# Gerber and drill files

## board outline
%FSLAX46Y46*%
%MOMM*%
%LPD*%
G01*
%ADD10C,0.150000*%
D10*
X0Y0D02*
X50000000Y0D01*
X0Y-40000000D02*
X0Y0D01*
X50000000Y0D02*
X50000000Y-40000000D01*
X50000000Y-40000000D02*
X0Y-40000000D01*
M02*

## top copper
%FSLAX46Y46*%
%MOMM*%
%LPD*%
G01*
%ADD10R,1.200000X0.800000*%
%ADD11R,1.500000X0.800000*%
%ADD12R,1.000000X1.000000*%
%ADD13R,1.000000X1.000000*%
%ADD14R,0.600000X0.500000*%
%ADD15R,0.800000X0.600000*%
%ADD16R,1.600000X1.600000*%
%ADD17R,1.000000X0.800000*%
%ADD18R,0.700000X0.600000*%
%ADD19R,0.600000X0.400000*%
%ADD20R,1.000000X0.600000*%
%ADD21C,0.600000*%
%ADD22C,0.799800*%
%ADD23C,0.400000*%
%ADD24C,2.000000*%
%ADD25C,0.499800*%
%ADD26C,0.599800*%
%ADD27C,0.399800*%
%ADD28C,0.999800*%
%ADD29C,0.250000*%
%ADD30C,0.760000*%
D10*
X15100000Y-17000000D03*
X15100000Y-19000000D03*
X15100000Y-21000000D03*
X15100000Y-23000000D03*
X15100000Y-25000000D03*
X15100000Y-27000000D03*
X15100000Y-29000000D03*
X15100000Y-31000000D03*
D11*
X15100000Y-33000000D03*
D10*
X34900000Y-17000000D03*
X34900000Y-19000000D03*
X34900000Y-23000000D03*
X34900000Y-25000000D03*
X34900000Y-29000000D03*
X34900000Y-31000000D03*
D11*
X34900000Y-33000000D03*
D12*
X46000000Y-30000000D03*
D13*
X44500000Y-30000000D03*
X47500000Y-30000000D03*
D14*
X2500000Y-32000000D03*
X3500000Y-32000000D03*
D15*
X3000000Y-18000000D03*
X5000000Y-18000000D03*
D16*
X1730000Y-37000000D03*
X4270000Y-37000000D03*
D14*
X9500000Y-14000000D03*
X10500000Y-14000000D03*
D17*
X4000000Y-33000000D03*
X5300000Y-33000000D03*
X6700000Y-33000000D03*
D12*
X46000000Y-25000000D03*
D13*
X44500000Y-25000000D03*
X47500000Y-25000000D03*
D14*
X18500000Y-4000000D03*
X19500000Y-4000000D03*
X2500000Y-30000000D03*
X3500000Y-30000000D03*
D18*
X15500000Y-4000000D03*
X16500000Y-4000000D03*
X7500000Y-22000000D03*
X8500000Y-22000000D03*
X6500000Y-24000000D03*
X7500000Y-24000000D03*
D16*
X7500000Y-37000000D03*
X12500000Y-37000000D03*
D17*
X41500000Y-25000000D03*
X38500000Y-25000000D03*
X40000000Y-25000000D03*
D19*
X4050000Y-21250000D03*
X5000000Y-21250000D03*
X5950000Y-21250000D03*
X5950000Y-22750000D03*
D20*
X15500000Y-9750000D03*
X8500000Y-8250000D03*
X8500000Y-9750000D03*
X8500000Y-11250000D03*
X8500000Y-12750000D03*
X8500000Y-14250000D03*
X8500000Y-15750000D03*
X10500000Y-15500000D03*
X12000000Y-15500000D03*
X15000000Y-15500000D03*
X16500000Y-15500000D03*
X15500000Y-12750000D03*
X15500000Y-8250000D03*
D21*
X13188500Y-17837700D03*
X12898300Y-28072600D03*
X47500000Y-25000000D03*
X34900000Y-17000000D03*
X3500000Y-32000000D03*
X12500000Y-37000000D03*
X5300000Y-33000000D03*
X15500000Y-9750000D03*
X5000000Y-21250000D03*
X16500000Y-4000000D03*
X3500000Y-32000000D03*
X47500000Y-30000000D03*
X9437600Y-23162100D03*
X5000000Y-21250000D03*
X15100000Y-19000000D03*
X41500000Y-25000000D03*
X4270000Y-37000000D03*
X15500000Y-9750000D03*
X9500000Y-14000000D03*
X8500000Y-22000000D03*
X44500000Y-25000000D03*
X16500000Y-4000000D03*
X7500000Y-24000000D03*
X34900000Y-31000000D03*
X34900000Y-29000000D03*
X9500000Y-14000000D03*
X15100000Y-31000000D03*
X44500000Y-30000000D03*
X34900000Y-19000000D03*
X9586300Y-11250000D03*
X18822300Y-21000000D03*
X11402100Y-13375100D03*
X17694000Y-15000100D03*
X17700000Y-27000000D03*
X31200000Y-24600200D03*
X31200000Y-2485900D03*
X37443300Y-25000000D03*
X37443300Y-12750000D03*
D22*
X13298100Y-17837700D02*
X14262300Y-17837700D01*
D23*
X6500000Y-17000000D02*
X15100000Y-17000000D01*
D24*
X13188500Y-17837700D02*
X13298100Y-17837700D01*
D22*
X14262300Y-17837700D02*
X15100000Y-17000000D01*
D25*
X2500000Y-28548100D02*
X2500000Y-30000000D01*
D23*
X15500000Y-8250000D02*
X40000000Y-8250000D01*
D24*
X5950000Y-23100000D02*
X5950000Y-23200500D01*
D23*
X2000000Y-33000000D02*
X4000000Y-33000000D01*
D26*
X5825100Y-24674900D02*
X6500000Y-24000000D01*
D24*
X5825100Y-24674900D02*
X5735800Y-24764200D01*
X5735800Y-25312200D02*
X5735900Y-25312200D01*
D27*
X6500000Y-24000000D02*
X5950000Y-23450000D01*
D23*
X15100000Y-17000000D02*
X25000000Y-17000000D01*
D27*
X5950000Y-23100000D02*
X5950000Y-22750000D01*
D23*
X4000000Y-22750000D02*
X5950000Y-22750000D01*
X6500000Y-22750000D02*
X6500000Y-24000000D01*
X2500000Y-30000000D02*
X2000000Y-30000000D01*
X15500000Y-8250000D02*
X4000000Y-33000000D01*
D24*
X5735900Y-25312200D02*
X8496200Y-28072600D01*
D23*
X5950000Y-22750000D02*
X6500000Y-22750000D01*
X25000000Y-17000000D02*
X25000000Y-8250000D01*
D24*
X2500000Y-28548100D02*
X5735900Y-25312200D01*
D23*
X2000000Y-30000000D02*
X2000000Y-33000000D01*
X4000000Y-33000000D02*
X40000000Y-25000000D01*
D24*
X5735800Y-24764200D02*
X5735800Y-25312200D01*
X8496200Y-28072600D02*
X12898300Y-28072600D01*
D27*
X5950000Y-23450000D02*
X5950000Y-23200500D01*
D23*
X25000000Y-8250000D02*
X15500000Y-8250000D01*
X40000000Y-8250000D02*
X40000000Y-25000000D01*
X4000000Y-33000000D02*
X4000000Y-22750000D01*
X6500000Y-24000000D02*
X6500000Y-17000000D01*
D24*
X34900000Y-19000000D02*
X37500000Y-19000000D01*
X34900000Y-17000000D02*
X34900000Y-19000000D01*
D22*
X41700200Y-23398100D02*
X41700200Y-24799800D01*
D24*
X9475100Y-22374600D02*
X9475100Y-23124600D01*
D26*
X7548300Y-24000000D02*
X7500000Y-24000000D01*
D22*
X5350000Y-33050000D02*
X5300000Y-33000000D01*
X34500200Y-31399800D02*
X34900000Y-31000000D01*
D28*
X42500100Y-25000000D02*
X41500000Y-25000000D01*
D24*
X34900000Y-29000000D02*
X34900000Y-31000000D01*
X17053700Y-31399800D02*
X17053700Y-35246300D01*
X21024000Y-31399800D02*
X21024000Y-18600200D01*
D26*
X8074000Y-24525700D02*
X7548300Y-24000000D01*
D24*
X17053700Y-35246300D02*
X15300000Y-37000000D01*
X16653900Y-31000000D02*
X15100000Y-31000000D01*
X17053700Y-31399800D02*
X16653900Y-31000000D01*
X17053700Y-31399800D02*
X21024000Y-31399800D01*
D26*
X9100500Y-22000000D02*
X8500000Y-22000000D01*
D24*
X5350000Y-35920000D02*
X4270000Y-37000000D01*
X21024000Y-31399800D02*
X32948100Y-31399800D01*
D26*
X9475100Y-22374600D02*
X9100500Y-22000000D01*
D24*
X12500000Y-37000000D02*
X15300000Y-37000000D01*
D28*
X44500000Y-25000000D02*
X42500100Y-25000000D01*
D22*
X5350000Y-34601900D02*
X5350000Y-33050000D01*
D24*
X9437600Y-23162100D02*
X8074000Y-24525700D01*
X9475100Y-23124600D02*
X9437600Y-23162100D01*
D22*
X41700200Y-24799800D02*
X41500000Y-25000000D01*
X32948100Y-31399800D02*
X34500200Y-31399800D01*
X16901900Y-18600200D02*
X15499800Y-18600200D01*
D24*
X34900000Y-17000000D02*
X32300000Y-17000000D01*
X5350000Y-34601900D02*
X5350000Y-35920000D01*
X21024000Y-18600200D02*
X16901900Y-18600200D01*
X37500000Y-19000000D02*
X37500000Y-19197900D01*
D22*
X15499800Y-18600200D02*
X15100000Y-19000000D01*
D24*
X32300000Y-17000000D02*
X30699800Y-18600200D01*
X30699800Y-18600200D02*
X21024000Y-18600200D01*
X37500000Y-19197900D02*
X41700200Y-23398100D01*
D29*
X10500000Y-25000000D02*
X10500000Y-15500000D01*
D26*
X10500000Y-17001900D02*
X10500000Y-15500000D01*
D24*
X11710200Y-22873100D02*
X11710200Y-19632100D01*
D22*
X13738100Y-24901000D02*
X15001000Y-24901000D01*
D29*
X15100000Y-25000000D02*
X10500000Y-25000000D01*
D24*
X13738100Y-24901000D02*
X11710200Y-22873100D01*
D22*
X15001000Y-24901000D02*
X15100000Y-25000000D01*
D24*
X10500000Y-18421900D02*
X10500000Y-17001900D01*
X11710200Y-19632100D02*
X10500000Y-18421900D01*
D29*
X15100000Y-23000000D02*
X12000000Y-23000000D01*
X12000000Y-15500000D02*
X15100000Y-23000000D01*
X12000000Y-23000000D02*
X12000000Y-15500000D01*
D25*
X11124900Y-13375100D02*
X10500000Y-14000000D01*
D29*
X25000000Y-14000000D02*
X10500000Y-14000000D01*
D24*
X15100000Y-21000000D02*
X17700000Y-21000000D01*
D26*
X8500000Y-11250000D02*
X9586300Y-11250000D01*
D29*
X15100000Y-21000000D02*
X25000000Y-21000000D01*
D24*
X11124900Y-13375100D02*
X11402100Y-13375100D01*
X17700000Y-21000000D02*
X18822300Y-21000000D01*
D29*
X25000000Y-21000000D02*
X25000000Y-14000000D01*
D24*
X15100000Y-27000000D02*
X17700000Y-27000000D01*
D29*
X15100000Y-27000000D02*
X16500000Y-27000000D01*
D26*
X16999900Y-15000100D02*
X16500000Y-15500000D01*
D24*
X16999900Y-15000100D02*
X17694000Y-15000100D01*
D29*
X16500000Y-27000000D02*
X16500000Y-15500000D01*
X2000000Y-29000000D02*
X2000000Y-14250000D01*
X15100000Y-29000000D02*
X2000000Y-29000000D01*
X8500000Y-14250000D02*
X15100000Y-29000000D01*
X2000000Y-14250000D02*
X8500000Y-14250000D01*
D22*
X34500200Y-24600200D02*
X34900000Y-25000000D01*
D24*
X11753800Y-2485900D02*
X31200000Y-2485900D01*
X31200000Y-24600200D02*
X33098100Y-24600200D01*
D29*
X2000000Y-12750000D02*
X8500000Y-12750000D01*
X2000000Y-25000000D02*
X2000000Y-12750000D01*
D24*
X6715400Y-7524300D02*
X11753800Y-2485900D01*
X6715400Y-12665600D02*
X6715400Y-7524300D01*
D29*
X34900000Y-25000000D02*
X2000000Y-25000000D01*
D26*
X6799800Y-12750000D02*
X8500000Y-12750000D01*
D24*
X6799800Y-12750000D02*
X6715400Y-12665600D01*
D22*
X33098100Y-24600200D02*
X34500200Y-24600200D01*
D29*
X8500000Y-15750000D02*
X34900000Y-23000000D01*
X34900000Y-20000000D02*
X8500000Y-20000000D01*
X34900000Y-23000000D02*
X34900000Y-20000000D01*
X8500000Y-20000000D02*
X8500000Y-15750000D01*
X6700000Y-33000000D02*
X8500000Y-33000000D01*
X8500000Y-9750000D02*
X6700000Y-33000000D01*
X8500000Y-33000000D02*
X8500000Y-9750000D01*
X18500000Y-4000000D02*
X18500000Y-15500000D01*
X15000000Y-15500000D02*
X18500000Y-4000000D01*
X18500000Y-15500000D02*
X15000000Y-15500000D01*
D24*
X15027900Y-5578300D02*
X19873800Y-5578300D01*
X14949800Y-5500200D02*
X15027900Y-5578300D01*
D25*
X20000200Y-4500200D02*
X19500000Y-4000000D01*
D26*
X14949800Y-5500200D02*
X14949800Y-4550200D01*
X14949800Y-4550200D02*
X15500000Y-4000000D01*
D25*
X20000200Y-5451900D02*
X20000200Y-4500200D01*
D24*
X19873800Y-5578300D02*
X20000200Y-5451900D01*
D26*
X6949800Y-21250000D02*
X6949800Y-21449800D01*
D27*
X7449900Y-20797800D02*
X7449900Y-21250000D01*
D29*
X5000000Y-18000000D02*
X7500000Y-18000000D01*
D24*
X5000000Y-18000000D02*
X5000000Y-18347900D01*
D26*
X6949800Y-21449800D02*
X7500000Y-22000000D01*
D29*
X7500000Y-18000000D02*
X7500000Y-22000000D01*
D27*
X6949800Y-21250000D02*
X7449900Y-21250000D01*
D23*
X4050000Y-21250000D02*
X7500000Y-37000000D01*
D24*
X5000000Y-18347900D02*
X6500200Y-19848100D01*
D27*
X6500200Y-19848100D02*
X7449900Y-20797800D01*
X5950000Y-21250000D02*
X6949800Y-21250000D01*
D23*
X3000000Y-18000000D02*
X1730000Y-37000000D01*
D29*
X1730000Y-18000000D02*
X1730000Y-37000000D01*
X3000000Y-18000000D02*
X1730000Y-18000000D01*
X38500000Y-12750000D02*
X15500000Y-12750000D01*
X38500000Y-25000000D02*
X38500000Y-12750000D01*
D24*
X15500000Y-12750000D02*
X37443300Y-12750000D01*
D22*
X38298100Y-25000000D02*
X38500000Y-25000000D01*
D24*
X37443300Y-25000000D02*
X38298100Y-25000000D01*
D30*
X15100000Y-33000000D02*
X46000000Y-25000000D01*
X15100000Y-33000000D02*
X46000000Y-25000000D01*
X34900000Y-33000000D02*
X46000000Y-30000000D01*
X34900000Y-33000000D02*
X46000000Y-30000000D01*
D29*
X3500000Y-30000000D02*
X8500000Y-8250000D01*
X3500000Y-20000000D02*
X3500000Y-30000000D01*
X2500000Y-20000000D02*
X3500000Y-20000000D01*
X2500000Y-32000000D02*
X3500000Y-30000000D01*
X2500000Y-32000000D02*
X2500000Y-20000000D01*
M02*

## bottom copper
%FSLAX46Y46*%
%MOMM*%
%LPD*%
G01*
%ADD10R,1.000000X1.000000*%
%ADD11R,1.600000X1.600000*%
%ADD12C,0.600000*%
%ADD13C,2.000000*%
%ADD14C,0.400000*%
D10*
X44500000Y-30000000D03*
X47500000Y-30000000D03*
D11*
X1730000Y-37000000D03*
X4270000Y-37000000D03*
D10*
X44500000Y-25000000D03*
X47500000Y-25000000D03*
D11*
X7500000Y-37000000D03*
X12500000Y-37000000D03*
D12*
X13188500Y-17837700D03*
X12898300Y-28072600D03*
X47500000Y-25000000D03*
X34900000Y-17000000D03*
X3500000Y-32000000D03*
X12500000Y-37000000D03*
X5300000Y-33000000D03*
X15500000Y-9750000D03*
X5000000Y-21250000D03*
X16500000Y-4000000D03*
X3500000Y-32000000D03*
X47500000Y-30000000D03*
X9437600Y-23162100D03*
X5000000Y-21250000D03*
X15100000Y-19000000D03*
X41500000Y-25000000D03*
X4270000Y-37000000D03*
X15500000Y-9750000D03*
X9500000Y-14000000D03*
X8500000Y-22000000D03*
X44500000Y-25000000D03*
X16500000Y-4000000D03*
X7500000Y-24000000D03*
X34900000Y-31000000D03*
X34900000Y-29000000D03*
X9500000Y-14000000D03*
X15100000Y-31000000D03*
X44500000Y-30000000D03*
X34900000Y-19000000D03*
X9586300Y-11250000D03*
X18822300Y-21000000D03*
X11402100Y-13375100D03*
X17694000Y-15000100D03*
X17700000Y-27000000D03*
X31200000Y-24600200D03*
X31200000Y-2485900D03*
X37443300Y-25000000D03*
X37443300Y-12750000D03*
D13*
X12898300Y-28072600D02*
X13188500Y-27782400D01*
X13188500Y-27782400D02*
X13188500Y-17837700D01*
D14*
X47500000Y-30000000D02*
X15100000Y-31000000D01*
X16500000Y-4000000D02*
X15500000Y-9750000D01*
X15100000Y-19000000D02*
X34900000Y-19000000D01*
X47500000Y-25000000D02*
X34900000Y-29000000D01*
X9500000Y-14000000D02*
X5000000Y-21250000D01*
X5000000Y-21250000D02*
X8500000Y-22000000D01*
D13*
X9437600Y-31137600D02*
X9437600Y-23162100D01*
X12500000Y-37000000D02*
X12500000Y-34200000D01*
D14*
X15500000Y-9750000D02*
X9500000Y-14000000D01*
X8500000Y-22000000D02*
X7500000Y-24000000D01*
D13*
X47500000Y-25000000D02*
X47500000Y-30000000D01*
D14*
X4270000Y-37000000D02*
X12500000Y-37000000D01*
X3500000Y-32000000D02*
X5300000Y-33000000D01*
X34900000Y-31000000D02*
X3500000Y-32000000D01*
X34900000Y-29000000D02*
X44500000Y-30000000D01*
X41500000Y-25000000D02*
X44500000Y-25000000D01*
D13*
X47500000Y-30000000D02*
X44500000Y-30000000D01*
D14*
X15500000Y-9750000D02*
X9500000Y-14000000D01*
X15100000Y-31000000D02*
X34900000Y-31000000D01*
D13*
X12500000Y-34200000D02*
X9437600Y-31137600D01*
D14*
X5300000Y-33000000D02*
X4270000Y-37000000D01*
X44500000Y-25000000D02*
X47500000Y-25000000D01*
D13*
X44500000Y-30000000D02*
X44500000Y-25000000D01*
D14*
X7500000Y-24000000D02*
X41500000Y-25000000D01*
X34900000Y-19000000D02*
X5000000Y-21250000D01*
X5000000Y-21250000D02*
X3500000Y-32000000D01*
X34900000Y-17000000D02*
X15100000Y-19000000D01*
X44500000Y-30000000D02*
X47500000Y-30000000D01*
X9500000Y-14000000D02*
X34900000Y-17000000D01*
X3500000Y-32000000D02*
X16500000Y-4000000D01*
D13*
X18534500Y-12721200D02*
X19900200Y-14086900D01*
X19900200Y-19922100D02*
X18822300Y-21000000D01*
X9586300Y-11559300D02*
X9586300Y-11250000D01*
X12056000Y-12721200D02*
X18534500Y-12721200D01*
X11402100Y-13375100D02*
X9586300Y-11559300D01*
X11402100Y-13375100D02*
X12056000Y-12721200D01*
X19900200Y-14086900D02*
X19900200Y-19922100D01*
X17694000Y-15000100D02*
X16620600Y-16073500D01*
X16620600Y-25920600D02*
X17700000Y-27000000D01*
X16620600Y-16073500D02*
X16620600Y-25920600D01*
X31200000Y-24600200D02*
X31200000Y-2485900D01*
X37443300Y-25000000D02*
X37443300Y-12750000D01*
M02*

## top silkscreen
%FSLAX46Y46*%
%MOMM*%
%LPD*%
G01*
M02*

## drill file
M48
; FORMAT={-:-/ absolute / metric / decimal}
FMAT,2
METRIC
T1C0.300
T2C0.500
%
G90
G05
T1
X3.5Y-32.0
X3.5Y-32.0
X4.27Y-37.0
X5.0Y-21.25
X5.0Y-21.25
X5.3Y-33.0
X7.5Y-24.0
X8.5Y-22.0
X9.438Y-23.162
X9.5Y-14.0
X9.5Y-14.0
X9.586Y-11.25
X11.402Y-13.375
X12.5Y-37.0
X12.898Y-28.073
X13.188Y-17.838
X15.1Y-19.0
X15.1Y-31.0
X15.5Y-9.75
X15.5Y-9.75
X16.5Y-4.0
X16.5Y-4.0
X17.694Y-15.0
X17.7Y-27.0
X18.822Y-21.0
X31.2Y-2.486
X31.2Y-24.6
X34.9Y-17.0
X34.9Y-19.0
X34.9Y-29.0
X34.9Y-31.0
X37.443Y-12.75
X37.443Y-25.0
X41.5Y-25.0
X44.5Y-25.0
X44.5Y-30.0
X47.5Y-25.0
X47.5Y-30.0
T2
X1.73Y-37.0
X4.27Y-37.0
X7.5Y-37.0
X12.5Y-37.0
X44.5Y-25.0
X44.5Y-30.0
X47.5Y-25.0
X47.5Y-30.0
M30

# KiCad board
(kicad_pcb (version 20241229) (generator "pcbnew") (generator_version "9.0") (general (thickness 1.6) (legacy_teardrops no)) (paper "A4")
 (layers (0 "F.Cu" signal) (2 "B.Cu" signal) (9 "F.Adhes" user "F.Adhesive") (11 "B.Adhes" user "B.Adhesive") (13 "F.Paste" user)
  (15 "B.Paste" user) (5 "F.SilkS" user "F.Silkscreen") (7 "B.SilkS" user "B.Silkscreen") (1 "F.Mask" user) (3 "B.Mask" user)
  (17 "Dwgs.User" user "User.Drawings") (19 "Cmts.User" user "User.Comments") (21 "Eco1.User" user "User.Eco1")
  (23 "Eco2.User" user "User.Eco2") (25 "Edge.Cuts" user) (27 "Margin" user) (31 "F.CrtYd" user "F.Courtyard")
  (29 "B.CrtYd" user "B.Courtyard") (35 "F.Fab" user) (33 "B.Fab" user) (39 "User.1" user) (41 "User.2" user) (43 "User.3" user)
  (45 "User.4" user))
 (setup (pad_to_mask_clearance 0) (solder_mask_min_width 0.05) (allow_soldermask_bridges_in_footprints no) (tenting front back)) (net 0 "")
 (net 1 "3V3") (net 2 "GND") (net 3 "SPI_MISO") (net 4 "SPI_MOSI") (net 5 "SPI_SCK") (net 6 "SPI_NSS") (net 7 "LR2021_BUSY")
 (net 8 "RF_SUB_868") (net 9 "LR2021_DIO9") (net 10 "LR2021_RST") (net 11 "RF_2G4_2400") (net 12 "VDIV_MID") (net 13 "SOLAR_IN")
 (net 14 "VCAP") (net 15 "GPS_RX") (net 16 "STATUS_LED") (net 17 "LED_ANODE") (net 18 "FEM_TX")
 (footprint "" (layer "F.Cu") (at 25 25)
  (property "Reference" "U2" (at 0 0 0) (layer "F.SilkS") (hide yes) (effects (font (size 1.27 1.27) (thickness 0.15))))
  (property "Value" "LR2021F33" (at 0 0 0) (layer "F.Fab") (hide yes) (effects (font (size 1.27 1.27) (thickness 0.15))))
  (pad "1" smd rect (at -9.9 -8) (size 1.2 0.8) (layers "F.Cu" "F.Mask") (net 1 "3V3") (thermal_bridge_angle 45))
  (pad "2" smd rect (at -9.9 -6) (size 1.2 0.8) (layers "F.Cu" "F.Mask") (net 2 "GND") (thermal_bridge_angle 45))
  (pad "3" smd rect (at -9.9 -4) (size 1.2 0.8) (layers "F.Cu" "F.Mask") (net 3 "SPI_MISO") (thermal_bridge_angle 45))
  (pad "4" smd rect (at -9.9 -2) (size 1.2 0.8) (layers "F.Cu" "F.Mask") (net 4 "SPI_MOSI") (thermal_bridge_angle 45))
  (pad "5" smd rect (at -9.9 0) (size 1.2 0.8) (layers "F.Cu" "F.Mask") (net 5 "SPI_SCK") (thermal_bridge_angle 45))
  (pad "6" smd rect (at -9.9 2) (size 1.2 0.8) (layers "F.Cu" "F.Mask") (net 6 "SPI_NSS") (thermal_bridge_angle 45))
  (pad "7" smd rect (at -9.9 4) (size 1.2 0.8) (layers "F.Cu" "F.Mask") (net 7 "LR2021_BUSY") (thermal_bridge_angle 45))
  (pad "8" smd rect (at -9.9 6) (size 1.2 0.8) (layers "F.Cu" "F.Mask") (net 2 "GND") (thermal_bridge_angle 45))
  (pad "9" smd rect (at -9.9 8) (size 1.5 0.8) (layers "F.Cu" "F.Mask") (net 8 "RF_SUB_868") (thermal_bridge_angle 45))
  (pad "10" smd rect (at 9.9 -8) (size 1.2 0.8) (layers "F.Cu" "F.Mask") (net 2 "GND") (thermal_bridge_angle 45))
  (pad "11" smd rect (at 9.9 -6) (size 1.2 0.8) (layers "F.Cu" "F.Mask") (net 2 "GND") (thermal_bridge_angle 45))
  (pad "13" smd rect (at 9.9 -2) (size 1.2 0.8) (layers "F.Cu" "F.Mask") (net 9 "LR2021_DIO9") (thermal_bridge_angle 45))
  (pad "14" smd rect (at 9.9 0) (size 1.2 0.8) (layers "F.Cu" "F.Mask") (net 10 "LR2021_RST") (thermal_bridge_angle 45))
  (pad "16" smd rect (at 9.9 4) (size 1.2 0.8) (layers "F.Cu" "F.Mask") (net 2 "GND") (thermal_bridge_angle 45))
  (pad "17" smd rect (at 9.9 6) (size 1.2 0.8) (layers "F.Cu" "F.Mask") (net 2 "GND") (thermal_bridge_angle 45))
  (pad "18" smd rect (at 9.9 8) (size 1.5 0.8) (layers "F.Cu" "F.Mask") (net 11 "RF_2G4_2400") (thermal_bridge_angle 45)))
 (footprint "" (layer "F.Cu") (at 46 30)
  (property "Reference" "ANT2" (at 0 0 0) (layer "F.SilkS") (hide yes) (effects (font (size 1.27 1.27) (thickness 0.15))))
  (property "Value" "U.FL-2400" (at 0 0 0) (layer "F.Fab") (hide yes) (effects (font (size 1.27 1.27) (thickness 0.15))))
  (pad "1" smd rect (at 0 0) (size 1 1) (layers "F.Cu" "F.Mask") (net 11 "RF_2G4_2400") (thermal_bridge_angle 45))
  (pad "2" thru_hole rect (at -1.5 0) (size 1 1) (drill 0.5) (layers "*.Cu" "*.Mask") (remove_unused_layers no) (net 2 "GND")
   (thermal_bridge_angle 45))
  (pad "3" thru_hole rect (at 1.5 0) (size 1 1) (drill 0.5) (layers "*.Cu" "*.Mask") (remove_unused_layers no) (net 2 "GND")
   (thermal_bridge_angle 45)))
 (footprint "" (layer "F.Cu") (at 3 32)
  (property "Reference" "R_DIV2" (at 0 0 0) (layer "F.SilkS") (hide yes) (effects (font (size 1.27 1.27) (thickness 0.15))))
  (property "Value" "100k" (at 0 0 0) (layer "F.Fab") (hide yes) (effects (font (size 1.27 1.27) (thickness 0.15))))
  (pad "1" smd rect (at -0.5 0) (size 0.6 0.5) (layers "F.Cu" "F.Mask") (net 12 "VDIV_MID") (thermal_bridge_angle 45))
  (pad "2" smd rect (at 0.5 0) (size 0.6 0.5) (layers "F.Cu" "F.Mask") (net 2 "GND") (thermal_bridge_angle 45)))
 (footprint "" (layer "F.Cu") (at 4 18)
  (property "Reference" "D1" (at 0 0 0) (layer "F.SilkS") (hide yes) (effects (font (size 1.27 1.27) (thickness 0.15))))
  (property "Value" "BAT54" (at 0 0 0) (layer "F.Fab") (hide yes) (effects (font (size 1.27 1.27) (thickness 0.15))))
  (pad "A" smd rect (at -1 0) (size 0.8 0.6) (layers "F.Cu" "F.Mask") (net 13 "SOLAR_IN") (thermal_bridge_angle 45))
  (pad "K" smd rect (at 1 0) (size 0.8 0.6) (layers "F.Cu" "F.Mask") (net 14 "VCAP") (thermal_bridge_angle 45)))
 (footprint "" (layer "F.Cu") (at 3 37)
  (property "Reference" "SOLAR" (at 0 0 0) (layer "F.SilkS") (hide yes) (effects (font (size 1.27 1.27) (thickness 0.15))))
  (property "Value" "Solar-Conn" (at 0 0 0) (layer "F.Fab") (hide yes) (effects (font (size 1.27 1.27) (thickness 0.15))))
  (pad "1" thru_hole rect (at -1.27 0) (size 1.6 1.6) (drill 0.5) (layers "*.Cu" "*.Mask") (remove_unused_layers no) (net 13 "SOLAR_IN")
   (thermal_bridge_angle 45))
  (pad "2" thru_hole rect (at 1.27 0) (size 1.6 1.6) (drill 0.5) (layers "*.Cu" "*.Mask") (remove_unused_layers no) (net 2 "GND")
   (thermal_bridge_angle 45)))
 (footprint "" (layer "F.Cu") (at 10 14)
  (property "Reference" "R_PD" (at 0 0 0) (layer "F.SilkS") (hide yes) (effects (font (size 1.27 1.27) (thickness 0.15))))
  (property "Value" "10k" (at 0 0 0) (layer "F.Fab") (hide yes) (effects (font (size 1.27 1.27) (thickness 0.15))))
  (pad "1" smd rect (at -0.5 0) (size 0.6 0.5) (layers "F.Cu" "F.Mask") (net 2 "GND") (thermal_bridge_angle 45))
  (pad "2" smd rect (at 0.5 0) (size 0.6 0.5) (layers "F.Cu" "F.Mask") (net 3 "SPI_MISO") (thermal_bridge_angle 45)))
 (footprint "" (layer "F.Cu") (at 6 33)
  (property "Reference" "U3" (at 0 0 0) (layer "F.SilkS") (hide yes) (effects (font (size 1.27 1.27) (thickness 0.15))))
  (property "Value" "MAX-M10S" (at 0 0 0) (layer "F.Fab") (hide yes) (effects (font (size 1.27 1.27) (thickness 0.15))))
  (pad "1" smd rect (at -2 0) (size 1 0.8) (layers "F.Cu" "F.Mask") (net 1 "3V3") (thermal_bridge_angle 45))
  (pad "2" smd rect (at -0.7 0) (size 1 0.8) (layers "F.Cu" "F.Mask") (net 2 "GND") (thermal_bridge_angle 45))
  (pad "3" smd rect (at 0.7 0) (size 1 0.8) (layers "F.Cu" "F.Mask") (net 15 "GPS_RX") (thermal_bridge_angle 45)))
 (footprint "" (layer "F.Cu") (at 46 25)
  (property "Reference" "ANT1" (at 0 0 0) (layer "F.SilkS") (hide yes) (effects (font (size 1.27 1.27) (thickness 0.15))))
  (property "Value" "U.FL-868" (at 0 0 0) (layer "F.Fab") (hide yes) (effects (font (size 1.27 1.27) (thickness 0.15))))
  (pad "1" smd rect (at 0 0) (size 1 1) (layers "F.Cu" "F.Mask") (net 8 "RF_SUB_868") (thermal_bridge_angle 45))
  (pad "2" thru_hole rect (at -1.5 0) (size 1 1) (drill 0.5) (layers "*.Cu" "*.Mask") (remove_unused_layers no) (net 2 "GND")
   (thermal_bridge_angle 45))
  (pad "3" thru_hole rect (at 1.5 0) (size 1 1) (drill 0.5) (layers "*.Cu" "*.Mask") (remove_unused_layers no) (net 2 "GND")
   (thermal_bridge_angle 45)))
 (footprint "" (layer "F.Cu") (at 19 4)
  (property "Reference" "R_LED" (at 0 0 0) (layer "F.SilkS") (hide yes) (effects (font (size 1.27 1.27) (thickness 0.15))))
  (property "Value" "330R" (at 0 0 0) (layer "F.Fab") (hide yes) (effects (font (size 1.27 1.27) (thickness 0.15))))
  (pad "1" smd rect (at -0.5 0) (size 0.6 0.5) (layers "F.Cu" "F.Mask") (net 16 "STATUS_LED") (thermal_bridge_angle 45))
  (pad "2" smd rect (at 0.5 0) (size 0.6 0.5) (layers "F.Cu" "F.Mask") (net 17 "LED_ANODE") (thermal_bridge_angle 45)))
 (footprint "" (layer "F.Cu") (at 3 30)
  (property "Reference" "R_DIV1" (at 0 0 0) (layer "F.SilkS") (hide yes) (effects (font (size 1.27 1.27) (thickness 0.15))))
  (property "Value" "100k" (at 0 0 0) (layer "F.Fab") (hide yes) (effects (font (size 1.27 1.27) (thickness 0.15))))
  (pad "1" smd rect (at -0.5 0) (size 0.6 0.5) (layers "F.Cu" "F.Mask") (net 1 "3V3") (thermal_bridge_angle 45))
  (pad "2" smd rect (at 0.5 0) (size 0.6 0.5) (layers "F.Cu" "F.Mask") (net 12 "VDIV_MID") (thermal_bridge_angle 45)))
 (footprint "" (layer "F.Cu") (at 16 4)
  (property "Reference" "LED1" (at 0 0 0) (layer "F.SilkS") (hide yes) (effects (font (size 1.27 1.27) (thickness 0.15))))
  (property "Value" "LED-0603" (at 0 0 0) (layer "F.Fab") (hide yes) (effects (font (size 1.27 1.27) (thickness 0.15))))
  (pad "A" smd rect (at -0.5 0) (size 0.7 0.6) (layers "F.Cu" "F.Mask") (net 17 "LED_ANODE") (thermal_bridge_angle 45))
  (pad "K" smd rect (at 0.5 0) (size 0.7 0.6) (layers "F.Cu" "F.Mask") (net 2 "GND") (thermal_bridge_angle 45)))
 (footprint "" (layer "F.Cu") (at 8 22)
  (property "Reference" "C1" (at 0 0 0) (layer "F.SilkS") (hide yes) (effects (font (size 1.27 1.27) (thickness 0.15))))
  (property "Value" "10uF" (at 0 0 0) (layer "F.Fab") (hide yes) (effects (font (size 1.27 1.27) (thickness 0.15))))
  (pad "1" smd rect (at -0.5 0) (size 0.7 0.6) (layers "F.Cu" "F.Mask") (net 14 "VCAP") (thermal_bridge_angle 45))
  (pad "2" smd rect (at 0.5 0) (size 0.7 0.6) (layers "F.Cu" "F.Mask") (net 2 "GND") (thermal_bridge_angle 45)))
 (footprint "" (layer "F.Cu") (at 7 24)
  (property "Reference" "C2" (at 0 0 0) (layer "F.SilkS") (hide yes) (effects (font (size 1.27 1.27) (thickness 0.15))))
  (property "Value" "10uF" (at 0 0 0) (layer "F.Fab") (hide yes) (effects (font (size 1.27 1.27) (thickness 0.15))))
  (pad "1" smd rect (at -0.5 0) (size 0.7 0.6) (layers "F.Cu" "F.Mask") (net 1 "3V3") (thermal_bridge_angle 45))
  (pad "2" smd rect (at 0.5 0) (size 0.7 0.6) (layers "F.Cu" "F.Mask") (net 2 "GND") (thermal_bridge_angle 45)))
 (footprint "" (layer "F.Cu") (at 10 37)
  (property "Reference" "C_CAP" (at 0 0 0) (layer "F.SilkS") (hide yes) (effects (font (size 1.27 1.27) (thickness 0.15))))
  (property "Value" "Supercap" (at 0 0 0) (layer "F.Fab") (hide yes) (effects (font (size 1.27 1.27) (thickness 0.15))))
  (pad "1" thru_hole rect (at -2.5 0) (size 1.6 1.6) (drill 0.5) (layers "*.Cu" "*.Mask") (remove_unused_layers no) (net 14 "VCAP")
   (thermal_bridge_angle 45))
  (pad "2" thru_hole rect (at 2.5 0) (size 1.6 1.6) (drill 0.5) (layers "*.Cu" "*.Mask") (remove_unused_layers no) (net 2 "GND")
   (thermal_bridge_angle 45)))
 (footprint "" (layer "F.Cu") (at 40 25)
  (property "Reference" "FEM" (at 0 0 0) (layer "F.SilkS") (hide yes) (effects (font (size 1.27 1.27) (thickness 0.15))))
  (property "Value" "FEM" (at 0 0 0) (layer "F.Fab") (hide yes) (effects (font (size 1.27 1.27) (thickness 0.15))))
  (pad "GND" smd rect (at 1.5 0) (size 1 0.8) (layers "F.Cu" "F.Mask") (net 2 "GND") (thermal_bridge_angle 45))
  (pad "TX" smd rect (at -1.5 0) (size 1 0.8) (layers "F.Cu" "F.Mask") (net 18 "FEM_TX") (thermal_bridge_angle 45))
  (pad "VCC" smd rect (at 0 0) (size 1 0.8) (layers "F.Cu" "F.Mask") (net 1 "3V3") (thermal_bridge_angle 45)))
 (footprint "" (layer "F.Cu") (at 5 22)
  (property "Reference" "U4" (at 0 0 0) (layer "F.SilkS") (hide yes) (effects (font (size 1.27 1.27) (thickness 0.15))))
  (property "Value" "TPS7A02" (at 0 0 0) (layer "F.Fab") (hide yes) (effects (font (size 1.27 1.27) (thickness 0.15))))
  (pad "1" smd rect (at -0.95 -0.75) (size 0.6 0.4) (layers "F.Cu" "F.Mask") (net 14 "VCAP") (thermal_bridge_angle 45))
  (pad "2" smd rect (at 0 -0.75) (size 0.6 0.4) (layers "F.Cu" "F.Mask") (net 2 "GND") (thermal_bridge_angle 45))
  (pad "3" smd rect (at 0.95 -0.75) (size 0.6 0.4) (layers "F.Cu" "F.Mask") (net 14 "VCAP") (thermal_bridge_angle 45))
  (pad "4" smd rect (at 0.95 0.75) (size 0.6 0.4) (layers "F.Cu" "F.Mask") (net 1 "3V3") (thermal_bridge_angle 45)))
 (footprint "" (layer "F.Cu") (at 12 12)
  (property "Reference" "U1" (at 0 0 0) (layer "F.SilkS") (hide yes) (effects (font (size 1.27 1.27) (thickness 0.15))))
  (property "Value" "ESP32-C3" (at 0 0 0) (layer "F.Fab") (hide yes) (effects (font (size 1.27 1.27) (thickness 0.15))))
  (pad "GND" smd rect (at 3.5 -2.25) (size 1 0.6) (layers "F.Cu" "F.Mask") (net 2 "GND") (thermal_bridge_angle 45))
  (pad "GPIO0" smd rect (at -3.5 -3.75) (size 1 0.6) (layers "F.Cu" "F.Mask") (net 12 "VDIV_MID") (thermal_bridge_angle 45))
  (pad "GPIO1" smd rect (at -3.5 -2.25) (size 1 0.6) (layers "F.Cu" "F.Mask") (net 15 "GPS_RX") (thermal_bridge_angle 45))
  (pad "GPIO2" smd rect (at -3.5 -0.75) (size 1 0.6) (layers "F.Cu" "F.Mask") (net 3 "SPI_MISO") (thermal_bridge_angle 45))
  (pad "GPIO3" smd rect (at -3.5 0.75) (size 1 0.6) (layers "F.Cu" "F.Mask") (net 10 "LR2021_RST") (thermal_bridge_angle 45))
  (pad "GPIO4" smd rect (at -3.5 2.25) (size 1 0.6) (layers "F.Cu" "F.Mask") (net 7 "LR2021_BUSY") (thermal_bridge_angle 45))
  (pad "GPIO5" smd rect (at -3.5 3.75) (size 1 0.6) (layers "F.Cu" "F.Mask") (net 9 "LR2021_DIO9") (thermal_bridge_angle 45))
  (pad "GPIO6" smd rect (at -1.5 3.5) (size 1 0.6) (layers "F.Cu" "F.Mask") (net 5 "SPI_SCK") (thermal_bridge_angle 45))
  (pad "GPIO7" smd rect (at 0 3.5) (size 1 0.6) (layers "F.Cu" "F.Mask") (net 4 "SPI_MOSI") (thermal_bridge_angle 45))
  (pad "GPIO9" smd rect (at 3 3.5) (size 1 0.6) (layers "F.Cu" "F.Mask") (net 16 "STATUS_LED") (thermal_bridge_angle 45))
  (pad "GPIO10" smd rect (at 4.5 3.5) (size 1 0.6) (layers "F.Cu" "F.Mask") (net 6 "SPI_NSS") (thermal_bridge_angle 45))
  (pad "GPIO19" smd rect (at 3.5 0.75) (size 1 0.6) (layers "F.Cu" "F.Mask") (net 18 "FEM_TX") (thermal_bridge_angle 45))
  (pad "VCC" smd rect (at 3.5 -3.75) (size 1 0.6) (layers "F.Cu" "F.Mask") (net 1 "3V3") (thermal_bridge_angle 45)))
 (gr_line (start 0 0) (end 50 0) (stroke (width 0.15) (type default)) (layer "Edge.Cuts"))
 (gr_line (start 0 40) (end 0 0) (stroke (width 0.15) (type default)) (layer "Edge.Cuts"))
 (gr_line (start 50 0) (end 50 40) (stroke (width 0.15) (type default)) (layer "Edge.Cuts"))
 (gr_line (start 50 40) (end 0 40) (stroke (width 0.15) (type default)) (layer "Edge.Cuts"))
 (segment (start 13.2981 17.8377) (end 14.2623 17.8377) (width 0.7998) (layer "F.Cu") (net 1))
 (segment (start 6.5 17) (end 15.1 17) (width 0.4) (layer "F.Cu") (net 1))
 (segment (start 13.1885 17.8377) (end 13.2981 17.8377) (width 2) (layer "F.Cu") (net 1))
 (segment (start 14.2623 17.8377) (end 15.1 17) (width 0.7998) (layer "F.Cu") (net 1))
 (segment (start 2.5 28.5481) (end 2.5 30) (width 0.4998) (layer "F.Cu") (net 1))
 (segment (start 15.5 8.25) (end 40 8.25) (width 0.4) (layer "F.Cu") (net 1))
 (segment (start 5.95 23.1) (end 5.95 23.2005) (width 2) (layer "F.Cu") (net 1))
 (segment (start 2 33) (end 4 33) (width 0.4) (layer "F.Cu") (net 1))
 (segment (start 5.8251 24.6749) (end 6.5 24) (width 0.5998) (layer "F.Cu") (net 1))
 (segment (start 5.8251 24.6749) (end 5.7358 24.7642) (width 2) (layer "F.Cu") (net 1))
 (segment (start 5.7358 25.3122) (end 5.7359 25.3122) (width 2) (layer "F.Cu") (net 1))
 (segment (start 6.5 24) (end 5.95 23.45) (width 0.3998) (layer "F.Cu") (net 1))
 (segment (start 15.1 17) (end 25 17) (width 0.4) (layer "F.Cu") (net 1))
 (segment (start 5.95 23.1) (end 5.95 22.75) (width 0.3998) (layer "F.Cu") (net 1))
 (segment (start 4 22.75) (end 5.95 22.75) (width 0.4) (layer "F.Cu") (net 1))
 (segment (start 6.5 22.75) (end 6.5 24) (width 0.4) (layer "F.Cu") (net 1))
 (segment (start 2.5 30) (end 2 30) (width 0.4) (layer "F.Cu") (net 1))
 (segment (start 15.5 8.25) (end 4 33) (width 0.4) (layer "F.Cu") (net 1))
 (segment (start 5.7359 25.3122) (end 8.4962 28.0726) (width 2) (layer "F.Cu") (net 1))
 (segment (start 5.95 22.75) (end 6.5 22.75) (width 0.4) (layer "F.Cu") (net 1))
 (segment (start 25 17) (end 25 8.25) (width 0.4) (layer "F.Cu") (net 1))
 (segment (start 2.5 28.5481) (end 5.7359 25.3122) (width 2) (layer "F.Cu") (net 1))
 (segment (start 2 30) (end 2 33) (width 0.4) (layer "F.Cu") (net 1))
 (segment (start 4 33) (end 40 25) (width 0.4) (layer "F.Cu") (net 1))
 (segment (start 5.7358 24.7642) (end 5.7358 25.3122) (width 2) (layer "F.Cu") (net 1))
 (segment (start 8.4962 28.0726) (end 12.8983 28.0726) (width 2) (layer "F.Cu") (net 1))
 (segment (start 5.95 23.45) (end 5.95 23.2005) (width 0.3998) (layer "F.Cu") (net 1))
 (segment (start 25 8.25) (end 15.5 8.25) (width 0.4) (layer "F.Cu") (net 1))
 (segment (start 40 8.25) (end 40 25) (width 0.4) (layer "F.Cu") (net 1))
 (segment (start 4 33) (end 4 22.75) (width 0.4) (layer "F.Cu") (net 1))
 (segment (start 6.5 24) (end 6.5 17) (width 0.4) (layer "F.Cu") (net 1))
 (via (at 13.1885 17.8377) (size 0.6) (drill 0.3) (layers "F.Cu" "B.Cu") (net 1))
 (via (at 12.8983 28.0726) (size 0.6) (drill 0.3) (layers "F.Cu" "B.Cu") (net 1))
 (segment (start 12.8983 28.0726) (end 13.1885 27.7824) (width 2) (layer "B.Cu") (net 1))
 (segment (start 13.1885 27.7824) (end 13.1885 17.8377) (width 2) (layer "B.Cu") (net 1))
 (segment (start 34.9 19) (end 37.5 19) (width 2) (layer "F.Cu") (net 2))
 (segment (start 34.9 17) (end 34.9 19) (width 2) (layer "F.Cu") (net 2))
 (segment (start 41.7002 23.3981) (end 41.7002 24.7998) (width 0.7998) (layer "F.Cu") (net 2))
 (segment (start 9.4751 22.3746) (end 9.4751 23.1246) (width 2) (layer "F.Cu") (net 2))
 (segment (start 7.5483 24) (end 7.5 24) (width 0.5998) (layer "F.Cu") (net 2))
 (segment (start 5.35 33.05) (end 5.3 33) (width 0.7998) (layer "F.Cu") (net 2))
 (segment (start 34.5002 31.3998) (end 34.9 31) (width 0.7998) (layer "F.Cu") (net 2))
 (segment (start 42.5001 25) (end 41.5 25) (width 0.9998) (layer "F.Cu") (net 2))
 (segment (start 34.9 29) (end 34.9 31) (width 2) (layer "F.Cu") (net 2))
 (segment (start 17.0537 31.3998) (end 17.0537 35.2463) (width 2) (layer "F.Cu") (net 2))
 (segment (start 21.024 31.3998) (end 21.024 18.6002) (width 2) (layer "F.Cu") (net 2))
 (segment (start 8.074 24.5257) (end 7.5483 24) (width 0.5998) (layer "F.Cu") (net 2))
 (segment (start 17.0537 35.2463) (end 15.3 37) (width 2) (layer "F.Cu") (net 2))
 (segment (start 16.6539 31) (end 15.1 31) (width 2) (layer "F.Cu") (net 2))
 (segment (start 17.0537 31.3998) (end 16.6539 31) (width 2) (layer "F.Cu") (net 2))
 (segment (start 17.0537 31.3998) (end 21.024 31.3998) (width 2) (layer "F.Cu") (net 2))
 (segment (start 9.1005 22) (end 8.5 22) (width 0.5998) (layer "F.Cu") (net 2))
 (segment (start 5.35 35.92) (end 4.27 37) (width 2) (layer "F.Cu") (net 2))
 (segment (start 21.024 31.3998) (end 32.9481 31.3998) (width 2) (layer "F.Cu") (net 2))
 (segment (start 9.4751 22.3746) (end 9.1005 22) (width 0.5998) (layer "F.Cu") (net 2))
 (segment (start 12.5 37) (end 15.3 37) (width 2) (layer "F.Cu") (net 2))
 (segment (start 44.5 25) (end 42.5001 25) (width 0.9998) (layer "F.Cu") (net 2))
 (segment (start 5.35 34.6019) (end 5.35 33.05) (width 0.7998) (layer "F.Cu") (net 2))
 (segment (start 9.4376 23.1621) (end 8.074 24.5257) (width 2) (layer "F.Cu") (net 2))
 (segment (start 9.4751 23.1246) (end 9.4376 23.1621) (width 2) (layer "F.Cu") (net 2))
 (segment (start 41.7002 24.7998) (end 41.5 25) (width 0.7998) (layer "F.Cu") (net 2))
 (segment (start 32.9481 31.3998) (end 34.5002 31.3998) (width 0.7998) (layer "F.Cu") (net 2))
 (segment (start 16.9019 18.6002) (end 15.4998 18.6002) (width 0.7998) (layer "F.Cu") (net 2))
 (segment (start 34.9 17) (end 32.3 17) (width 2) (layer "F.Cu") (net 2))
 (segment (start 5.35 34.6019) (end 5.35 35.92) (width 2) (layer "F.Cu") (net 2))
 (segment (start 21.024 18.6002) (end 16.9019 18.6002) (width 2) (layer "F.Cu") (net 2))
 (segment (start 37.5 19) (end 37.5 19.1979) (width 2) (layer "F.Cu") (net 2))
 (segment (start 15.4998 18.6002) (end 15.1 19) (width 0.7998) (layer "F.Cu") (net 2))
 (segment (start 32.3 17) (end 30.6998 18.6002) (width 2) (layer "F.Cu") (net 2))
 (segment (start 30.6998 18.6002) (end 21.024 18.6002) (width 2) (layer "F.Cu") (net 2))
 (segment (start 37.5 19.1979) (end 41.7002 23.3981) (width 2) (layer "F.Cu") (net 2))
 (via (at 47.5 25) (size 0.6) (drill 0.3) (layers "F.Cu" "B.Cu") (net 2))
 (via (at 34.9 17) (size 0.6) (drill 0.3) (layers "F.Cu" "B.Cu") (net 2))
 (via (at 3.5 32) (size 0.6) (drill 0.3) (layers "F.Cu" "B.Cu") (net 2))
 (via (at 12.5 37) (size 0.6) (drill 0.3) (layers "F.Cu" "B.Cu") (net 2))
 (via (at 5.3 33) (size 0.6) (drill 0.3) (layers "F.Cu" "B.Cu") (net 2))
 (via (at 15.5 9.75) (size 0.6) (drill 0.3) (layers "F.Cu" "B.Cu") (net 2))
 (via (at 5 21.25) (size 0.6) (drill 0.3) (layers "F.Cu" "B.Cu") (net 2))
 (via (at 16.5 4) (size 0.6) (drill 0.3) (layers "F.Cu" "B.Cu") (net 2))
 (via (at 3.5 32) (size 0.6) (drill 0.3) (layers "F.Cu" "B.Cu") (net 2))
 (via (at 47.5 30) (size 0.6) (drill 0.3) (layers "F.Cu" "B.Cu") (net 2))
 (via (at 9.4376 23.1621) (size 0.6) (drill 0.3) (layers "F.Cu" "B.Cu") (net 2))
 (via (at 5 21.25) (size 0.6) (drill 0.3) (layers "F.Cu" "B.Cu") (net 2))
 (via (at 15.1 19) (size 0.6) (drill 0.3) (layers "F.Cu" "B.Cu") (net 2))
 (via (at 41.5 25) (size 0.6) (drill 0.3) (layers "F.Cu" "B.Cu") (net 2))
 (via (at 4.27 37) (size 0.6) (drill 0.3) (layers "F.Cu" "B.Cu") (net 2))
 (via (at 15.5 9.75) (size 0.6) (drill 0.3) (layers "F.Cu" "B.Cu") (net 2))
 (via (at 9.5 14) (size 0.6) (drill 0.3) (layers "F.Cu" "B.Cu") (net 2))
 (via (at 8.5 22) (size 0.6) (drill 0.3) (layers "F.Cu" "B.Cu") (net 2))
 (via (at 44.5 25) (size 0.6) (drill 0.3) (layers "F.Cu" "B.Cu") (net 2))
 (via (at 16.5 4) (size 0.6) (drill 0.3) (layers "F.Cu" "B.Cu") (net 2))
 (via (at 7.5 24) (size 0.6) (drill 0.3) (layers "F.Cu" "B.Cu") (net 2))
 (via (at 34.9 31) (size 0.6) (drill 0.3) (layers "F.Cu" "B.Cu") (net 2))
 (via (at 34.9 29) (size 0.6) (drill 0.3) (layers "F.Cu" "B.Cu") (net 2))
 (via (at 9.5 14) (size 0.6) (drill 0.3) (layers "F.Cu" "B.Cu") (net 2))
 (via (at 15.1 31) (size 0.6) (drill 0.3) (layers "F.Cu" "B.Cu") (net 2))
 (via (at 44.5 30) (size 0.6) (drill 0.3) (layers "F.Cu" "B.Cu") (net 2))
 (via (at 34.9 19) (size 0.6) (drill 0.3) (layers "F.Cu" "B.Cu") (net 2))
 (segment (start 47.5 30) (end 15.1 31) (width 0.4) (layer "B.Cu") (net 2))
 (segment (start 16.5 4) (end 15.5 9.75) (width 0.4) (layer "B.Cu") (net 2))
 (segment (start 15.1 19) (end 34.9 19) (width 0.4) (layer "B.Cu") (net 2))
 (segment (start 47.5 25) (end 34.9 29) (width 0.4) (layer "B.Cu") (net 2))
 (segment (start 9.5 14) (end 5 21.25) (width 0.4) (layer "B.Cu") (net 2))
 (segment (start 5 21.25) (end 8.5 22) (width 0.4) (layer "B.Cu") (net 2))
 (segment (start 9.4376 31.1376) (end 9.4376 23.1621) (width 2) (layer "B.Cu") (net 2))
 (segment (start 12.5 37) (end 12.5 34.2) (width 2) (layer "B.Cu") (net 2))
 (segment (start 15.5 9.75) (end 9.5 14) (width 0.4) (layer "B.Cu") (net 2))
 (segment (start 8.5 22) (end 7.5 24) (width 0.4) (layer "B.Cu") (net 2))
 (segment (start 47.5 25) (end 47.5 30) (width 2) (layer "B.Cu") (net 2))
 (segment (start 4.27 37) (end 12.5 37) (width 0.4) (layer "B.Cu") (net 2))
 (segment (start 3.5 32) (end 5.3 33) (width 0.4) (layer "B.Cu") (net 2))
 (segment (start 34.9 31) (end 3.5 32) (width 0.4) (layer "B.Cu") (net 2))
 (segment (start 34.9 29) (end 44.5 30) (width 0.4) (layer "B.Cu") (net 2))
 (segment (start 41.5 25) (end 44.5 25) (width 0.4) (layer "B.Cu") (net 2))
 (segment (start 47.5 30) (end 44.5 30) (width 2) (layer "B.Cu") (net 2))
 (segment (start 15.5 9.75) (end 9.5 14) (width 0.4) (layer "B.Cu") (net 2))
 (segment (start 15.1 31) (end 34.9 31) (width 0.4) (layer "B.Cu") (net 2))
 (segment (start 12.5 34.2) (end 9.4376 31.1376) (width 2) (layer "B.Cu") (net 2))
 (segment (start 5.3 33) (end 4.27 37) (width 0.4) (layer "B.Cu") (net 2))
 (segment (start 44.5 25) (end 47.5 25) (width 0.4) (layer "B.Cu") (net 2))
 (segment (start 44.5 30) (end 44.5 25) (width 2) (layer "B.Cu") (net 2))
 (segment (start 7.5 24) (end 41.5 25) (width 0.4) (layer "B.Cu") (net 2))
 (segment (start 34.9 19) (end 5 21.25) (width 0.4) (layer "B.Cu") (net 2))
 (segment (start 5 21.25) (end 3.5 32) (width 0.4) (layer "B.Cu") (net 2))
 (segment (start 34.9 17) (end 15.1 19) (width 0.4) (layer "B.Cu") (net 2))
 (segment (start 44.5 30) (end 47.5 30) (width 0.4) (layer "B.Cu") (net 2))
 (segment (start 9.5 14) (end 34.9 17) (width 0.4) (layer "B.Cu") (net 2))
 (segment (start 3.5 32) (end 16.5 4) (width 0.4) (layer "B.Cu") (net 2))
 (segment (start 10.5 25) (end 10.5 15.5) (width 0.25) (layer "F.Cu") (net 5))
 (segment (start 10.5 17.0019) (end 10.5 15.5) (width 0.5998) (layer "F.Cu") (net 5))
 (segment (start 11.7102 22.8731) (end 11.7102 19.6321) (width 2) (layer "F.Cu") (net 5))
 (segment (start 13.7381 24.901) (end 15.001 24.901) (width 0.7998) (layer "F.Cu") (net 5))
 (segment (start 15.1 25) (end 10.5 25) (width 0.25) (layer "F.Cu") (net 5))
 (segment (start 13.7381 24.901) (end 11.7102 22.8731) (width 2) (layer "F.Cu") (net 5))
 (segment (start 15.001 24.901) (end 15.1 25) (width 0.7998) (layer "F.Cu") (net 5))
 (segment (start 10.5 18.4219) (end 10.5 17.0019) (width 2) (layer "F.Cu") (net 5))
 (segment (start 11.7102 19.6321) (end 10.5 18.4219) (width 2) (layer "F.Cu") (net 5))
 (segment (start 15.1 23) (end 12 23) (width 0.25) (layer "F.Cu") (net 4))
 (segment (start 12 15.5) (end 15.1 23) (width 0.25) (layer "F.Cu") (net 4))
 (segment (start 12 23) (end 12 15.5) (width 0.25) (layer "F.Cu") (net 4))
 (segment (start 11.1249 13.3751) (end 10.5 14) (width 0.4998) (layer "F.Cu") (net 3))
 (segment (start 25 14) (end 10.5 14) (width 0.25) (layer "F.Cu") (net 3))
 (segment (start 15.1 21) (end 17.7 21) (width 2) (layer "F.Cu") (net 3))
 (segment (start 8.5 11.25) (end 9.5863 11.25) (width 0.5998) (layer "F.Cu") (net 3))
 (segment (start 15.1 21) (end 25 21) (width 0.25) (layer "F.Cu") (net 3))
 (segment (start 11.1249 13.3751) (end 11.4021 13.3751) (width 2) (layer "F.Cu") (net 3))
 (segment (start 17.7 21) (end 18.8223 21) (width 2) (layer "F.Cu") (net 3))
 (segment (start 25 21) (end 25 14) (width 0.25) (layer "F.Cu") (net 3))
 (via (at 9.5863 11.25) (size 0.6) (drill 0.3) (layers "F.Cu" "B.Cu") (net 3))
 (via (at 18.8223 21) (size 0.6) (drill 0.3) (layers "F.Cu" "B.Cu") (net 3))
 (via (at 11.4021 13.3751) (size 0.6) (drill 0.3) (layers "F.Cu" "B.Cu") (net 3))
 (segment (start 18.5345 12.7212) (end 19.9002 14.0869) (width 2) (layer "B.Cu") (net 3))
 (segment (start 19.9002 19.9221) (end 18.8223 21) (width 2) (layer "B.Cu") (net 3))
 (segment (start 9.5863 11.5593) (end 9.5863 11.25) (width 2) (layer "B.Cu") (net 3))
 (segment (start 12.056 12.7212) (end 18.5345 12.7212) (width 2) (layer "B.Cu") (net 3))
 (segment (start 11.4021 13.3751) (end 9.5863 11.5593) (width 2) (layer "B.Cu") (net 3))
 (segment (start 11.4021 13.3751) (end 12.056 12.7212) (width 2) (layer "B.Cu") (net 3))
 (segment (start 19.9002 14.0869) (end 19.9002 19.9221) (width 2) (layer "B.Cu") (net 3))
 (segment (start 15.1 27) (end 17.7 27) (width 2) (layer "F.Cu") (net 6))
 (segment (start 15.1 27) (end 16.5 27) (width 0.25) (layer "F.Cu") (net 6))
 (segment (start 16.9999 15.0001) (end 16.5 15.5) (width 0.5998) (layer "F.Cu") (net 6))
 (segment (start 16.9999 15.0001) (end 17.694 15.0001) (width 2) (layer "F.Cu") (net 6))
 (segment (start 16.5 27) (end 16.5 15.5) (width 0.25) (layer "F.Cu") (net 6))
 (via (at 17.694 15.0001) (size 0.6) (drill 0.3) (layers "F.Cu" "B.Cu") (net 6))
 (via (at 17.7 27) (size 0.6) (drill 0.3) (layers "F.Cu" "B.Cu") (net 6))
 (segment (start 17.694 15.0001) (end 16.6206 16.0735) (width 2) (layer "B.Cu") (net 6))
 (segment (start 16.6206 25.9206) (end 17.7 27) (width 2) (layer "B.Cu") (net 6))
 (segment (start 16.6206 16.0735) (end 16.6206 25.9206) (width 2) (layer "B.Cu") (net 6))
 (segment (start 2 29) (end 2 14.25) (width 0.25) (layer "F.Cu") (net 7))
 (segment (start 15.1 29) (end 2 29) (width 0.25) (layer "F.Cu") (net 7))
 (segment (start 8.5 14.25) (end 15.1 29) (width 0.25) (layer "F.Cu") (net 7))
 (segment (start 2 14.25) (end 8.5 14.25) (width 0.25) (layer "F.Cu") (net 7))
 (segment (start 34.5002 24.6002) (end 34.9 25) (width 0.7998) (layer "F.Cu") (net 10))
 (segment (start 11.7538 2.4859) (end 31.2 2.4859) (width 2) (layer "F.Cu") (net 10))
 (segment (start 31.2 24.6002) (end 33.0981 24.6002) (width 2) (layer "F.Cu") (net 10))
 (segment (start 2 12.75) (end 8.5 12.75) (width 0.25) (layer "F.Cu") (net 10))
 (segment (start 2 25) (end 2 12.75) (width 0.25) (layer "F.Cu") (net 10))
 (segment (start 6.7154 7.5243) (end 11.7538 2.4859) (width 2) (layer "F.Cu") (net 10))
 (segment (start 6.7154 12.6656) (end 6.7154 7.5243) (width 2) (layer "F.Cu") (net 10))
 (segment (start 34.9 25) (end 2 25) (width 0.25) (layer "F.Cu") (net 10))
 (segment (start 6.7998 12.75) (end 8.5 12.75) (width 0.5998) (layer "F.Cu") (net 10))
 (segment (start 6.7998 12.75) (end 6.7154 12.6656) (width 2) (layer "F.Cu") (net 10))
 (segment (start 33.0981 24.6002) (end 34.5002 24.6002) (width 0.7998) (layer "F.Cu") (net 10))
 (via (at 31.2 24.6002) (size 0.6) (drill 0.3) (layers "F.Cu" "B.Cu") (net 10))
 (via (at 31.2 2.4859) (size 0.6) (drill 0.3) (layers "F.Cu" "B.Cu") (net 10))
 (segment (start 31.2 24.6002) (end 31.2 2.4859) (width 2) (layer "B.Cu") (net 10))
 (segment (start 8.5 15.75) (end 34.9 23) (width 0.25) (layer "F.Cu") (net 9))
 (segment (start 34.9 20) (end 8.5 20) (width 0.25) (layer "F.Cu") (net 9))
 (segment (start 34.9 23) (end 34.9 20) (width 0.25) (layer "F.Cu") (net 9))
 (segment (start 8.5 20) (end 8.5 15.75) (width 0.25) (layer "F.Cu") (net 9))
 (segment (start 6.7 33) (end 8.5 33) (width 0.25) (layer "F.Cu") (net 15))
 (segment (start 8.5 9.75) (end 6.7 33) (width 0.25) (layer "F.Cu") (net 15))
 (segment (start 8.5 33) (end 8.5 9.75) (width 0.25) (layer "F.Cu") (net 15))
 (segment (start 18.5 4) (end 18.5 15.5) (width 0.25) (layer "F.Cu") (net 16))
 (segment (start 15 15.5) (end 18.5 4) (width 0.25) (layer "F.Cu") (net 16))
 (segment (start 18.5 15.5) (end 15 15.5) (width 0.25) (layer "F.Cu") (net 16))
 (segment (start 15.0279 5.5783) (end 19.8738 5.5783) (width 2) (layer "F.Cu") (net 17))
 (segment (start 14.9498 5.5002) (end 15.0279 5.5783) (width 2) (layer "F.Cu") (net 17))
 (segment (start 20.0002 4.5002) (end 19.5 4) (width 0.4998) (layer "F.Cu") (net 17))
 (segment (start 14.9498 5.5002) (end 14.9498 4.5502) (width 0.5998) (layer "F.Cu") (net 17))
 (segment (start 14.9498 4.5502) (end 15.5 4) (width 0.5998) (layer "F.Cu") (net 17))
 (segment (start 20.0002 5.4519) (end 20.0002 4.5002) (width 0.4998) (layer "F.Cu") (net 17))
 (segment (start 19.8738 5.5783) (end 20.0002 5.4519) (width 2) (layer "F.Cu") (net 17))
 (segment (start 6.9498 21.25) (end 6.9498 21.4498) (width 0.5998) (layer "F.Cu") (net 14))
 (segment (start 7.4499 20.7978) (end 7.4499 21.25) (width 0.3998) (layer "F.Cu") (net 14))
 (segment (start 5 18) (end 7.5 18) (width 0.25) (layer "F.Cu") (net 14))
 (segment (start 5 18) (end 5 18.3479) (width 2) (layer "F.Cu") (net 14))
 (segment (start 6.9498 21.4498) (end 7.5 22) (width 0.5998) (layer "F.Cu") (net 14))
 (segment (start 7.5 18) (end 7.5 22) (width 0.25) (layer "F.Cu") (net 14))
 (segment (start 6.9498 21.25) (end 7.4499 21.25) (width 0.3998) (layer "F.Cu") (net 14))
 (segment (start 4.05 21.25) (end 7.5 37) (width 0.4) (layer "F.Cu") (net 14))
 (segment (start 5 18.3479) (end 6.5002 19.8481) (width 2) (layer "F.Cu") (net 14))
 (segment (start 6.5002 19.8481) (end 7.4499 20.7978) (width 0.3998) (layer "F.Cu") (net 14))
 (segment (start 5.95 21.25) (end 6.9498 21.25) (width 0.3998) (layer "F.Cu") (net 14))
 (segment (start 3 18) (end 1.73 37) (width 0.4) (layer "F.Cu") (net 13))
 (segment (start 1.73 18) (end 1.73 37) (width 0.25) (layer "F.Cu") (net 13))
 (segment (start 3 18) (end 1.73 18) (width 0.25) (layer "F.Cu") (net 13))
 (segment (start 38.5 12.75) (end 15.5 12.75) (width 0.25) (layer "F.Cu") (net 18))
 (segment (start 38.5 25) (end 38.5 12.75) (width 0.25) (layer "F.Cu") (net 18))
 (segment (start 15.5 12.75) (end 37.4433 12.75) (width 2) (layer "F.Cu") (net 18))
 (segment (start 38.2981 25) (end 38.5 25) (width 0.7998) (layer "F.Cu") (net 18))
 (segment (start 37.4433 25) (end 38.2981 25) (width 2) (layer "F.Cu") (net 18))
 (via (at 37.4433 25) (size 0.6) (drill 0.3) (layers "F.Cu" "B.Cu") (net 18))
 (via (at 37.4433 12.75) (size 0.6) (drill 0.3) (layers "F.Cu" "B.Cu") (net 18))
 (segment (start 37.4433 25) (end 37.4433 12.75) (width 2) (layer "B.Cu") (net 18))
 (segment (start 15.1 33) (end 46 25) (width 0.76) (layer "F.Cu") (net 8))
 (segment (start 15.1 33) (end 46 25) (width 0.76) (layer "F.Cu") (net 8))
 (segment (start 34.9 33) (end 46 30) (width 0.76) (layer "F.Cu") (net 11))
 (segment (start 34.9 33) (end 46 30) (width 0.76) (layer "F.Cu") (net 11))
 (segment (start 3.5 30) (end 8.5 8.25) (width 0.25) (layer "F.Cu") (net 12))
 (segment (start 3.5 20) (end 3.5 30) (width 0.25) (layer "F.Cu") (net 12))
 (segment (start 2.5 20) (end 3.5 20) (width 0.25) (layer "F.Cu") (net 12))
 (segment (start 2.5 32) (end 3.5 30) (width 0.25) (layer "F.Cu") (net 12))
 (segment (start 2.5 32) (end 2.5 20) (width 0.25) (layer "F.Cu") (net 12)))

